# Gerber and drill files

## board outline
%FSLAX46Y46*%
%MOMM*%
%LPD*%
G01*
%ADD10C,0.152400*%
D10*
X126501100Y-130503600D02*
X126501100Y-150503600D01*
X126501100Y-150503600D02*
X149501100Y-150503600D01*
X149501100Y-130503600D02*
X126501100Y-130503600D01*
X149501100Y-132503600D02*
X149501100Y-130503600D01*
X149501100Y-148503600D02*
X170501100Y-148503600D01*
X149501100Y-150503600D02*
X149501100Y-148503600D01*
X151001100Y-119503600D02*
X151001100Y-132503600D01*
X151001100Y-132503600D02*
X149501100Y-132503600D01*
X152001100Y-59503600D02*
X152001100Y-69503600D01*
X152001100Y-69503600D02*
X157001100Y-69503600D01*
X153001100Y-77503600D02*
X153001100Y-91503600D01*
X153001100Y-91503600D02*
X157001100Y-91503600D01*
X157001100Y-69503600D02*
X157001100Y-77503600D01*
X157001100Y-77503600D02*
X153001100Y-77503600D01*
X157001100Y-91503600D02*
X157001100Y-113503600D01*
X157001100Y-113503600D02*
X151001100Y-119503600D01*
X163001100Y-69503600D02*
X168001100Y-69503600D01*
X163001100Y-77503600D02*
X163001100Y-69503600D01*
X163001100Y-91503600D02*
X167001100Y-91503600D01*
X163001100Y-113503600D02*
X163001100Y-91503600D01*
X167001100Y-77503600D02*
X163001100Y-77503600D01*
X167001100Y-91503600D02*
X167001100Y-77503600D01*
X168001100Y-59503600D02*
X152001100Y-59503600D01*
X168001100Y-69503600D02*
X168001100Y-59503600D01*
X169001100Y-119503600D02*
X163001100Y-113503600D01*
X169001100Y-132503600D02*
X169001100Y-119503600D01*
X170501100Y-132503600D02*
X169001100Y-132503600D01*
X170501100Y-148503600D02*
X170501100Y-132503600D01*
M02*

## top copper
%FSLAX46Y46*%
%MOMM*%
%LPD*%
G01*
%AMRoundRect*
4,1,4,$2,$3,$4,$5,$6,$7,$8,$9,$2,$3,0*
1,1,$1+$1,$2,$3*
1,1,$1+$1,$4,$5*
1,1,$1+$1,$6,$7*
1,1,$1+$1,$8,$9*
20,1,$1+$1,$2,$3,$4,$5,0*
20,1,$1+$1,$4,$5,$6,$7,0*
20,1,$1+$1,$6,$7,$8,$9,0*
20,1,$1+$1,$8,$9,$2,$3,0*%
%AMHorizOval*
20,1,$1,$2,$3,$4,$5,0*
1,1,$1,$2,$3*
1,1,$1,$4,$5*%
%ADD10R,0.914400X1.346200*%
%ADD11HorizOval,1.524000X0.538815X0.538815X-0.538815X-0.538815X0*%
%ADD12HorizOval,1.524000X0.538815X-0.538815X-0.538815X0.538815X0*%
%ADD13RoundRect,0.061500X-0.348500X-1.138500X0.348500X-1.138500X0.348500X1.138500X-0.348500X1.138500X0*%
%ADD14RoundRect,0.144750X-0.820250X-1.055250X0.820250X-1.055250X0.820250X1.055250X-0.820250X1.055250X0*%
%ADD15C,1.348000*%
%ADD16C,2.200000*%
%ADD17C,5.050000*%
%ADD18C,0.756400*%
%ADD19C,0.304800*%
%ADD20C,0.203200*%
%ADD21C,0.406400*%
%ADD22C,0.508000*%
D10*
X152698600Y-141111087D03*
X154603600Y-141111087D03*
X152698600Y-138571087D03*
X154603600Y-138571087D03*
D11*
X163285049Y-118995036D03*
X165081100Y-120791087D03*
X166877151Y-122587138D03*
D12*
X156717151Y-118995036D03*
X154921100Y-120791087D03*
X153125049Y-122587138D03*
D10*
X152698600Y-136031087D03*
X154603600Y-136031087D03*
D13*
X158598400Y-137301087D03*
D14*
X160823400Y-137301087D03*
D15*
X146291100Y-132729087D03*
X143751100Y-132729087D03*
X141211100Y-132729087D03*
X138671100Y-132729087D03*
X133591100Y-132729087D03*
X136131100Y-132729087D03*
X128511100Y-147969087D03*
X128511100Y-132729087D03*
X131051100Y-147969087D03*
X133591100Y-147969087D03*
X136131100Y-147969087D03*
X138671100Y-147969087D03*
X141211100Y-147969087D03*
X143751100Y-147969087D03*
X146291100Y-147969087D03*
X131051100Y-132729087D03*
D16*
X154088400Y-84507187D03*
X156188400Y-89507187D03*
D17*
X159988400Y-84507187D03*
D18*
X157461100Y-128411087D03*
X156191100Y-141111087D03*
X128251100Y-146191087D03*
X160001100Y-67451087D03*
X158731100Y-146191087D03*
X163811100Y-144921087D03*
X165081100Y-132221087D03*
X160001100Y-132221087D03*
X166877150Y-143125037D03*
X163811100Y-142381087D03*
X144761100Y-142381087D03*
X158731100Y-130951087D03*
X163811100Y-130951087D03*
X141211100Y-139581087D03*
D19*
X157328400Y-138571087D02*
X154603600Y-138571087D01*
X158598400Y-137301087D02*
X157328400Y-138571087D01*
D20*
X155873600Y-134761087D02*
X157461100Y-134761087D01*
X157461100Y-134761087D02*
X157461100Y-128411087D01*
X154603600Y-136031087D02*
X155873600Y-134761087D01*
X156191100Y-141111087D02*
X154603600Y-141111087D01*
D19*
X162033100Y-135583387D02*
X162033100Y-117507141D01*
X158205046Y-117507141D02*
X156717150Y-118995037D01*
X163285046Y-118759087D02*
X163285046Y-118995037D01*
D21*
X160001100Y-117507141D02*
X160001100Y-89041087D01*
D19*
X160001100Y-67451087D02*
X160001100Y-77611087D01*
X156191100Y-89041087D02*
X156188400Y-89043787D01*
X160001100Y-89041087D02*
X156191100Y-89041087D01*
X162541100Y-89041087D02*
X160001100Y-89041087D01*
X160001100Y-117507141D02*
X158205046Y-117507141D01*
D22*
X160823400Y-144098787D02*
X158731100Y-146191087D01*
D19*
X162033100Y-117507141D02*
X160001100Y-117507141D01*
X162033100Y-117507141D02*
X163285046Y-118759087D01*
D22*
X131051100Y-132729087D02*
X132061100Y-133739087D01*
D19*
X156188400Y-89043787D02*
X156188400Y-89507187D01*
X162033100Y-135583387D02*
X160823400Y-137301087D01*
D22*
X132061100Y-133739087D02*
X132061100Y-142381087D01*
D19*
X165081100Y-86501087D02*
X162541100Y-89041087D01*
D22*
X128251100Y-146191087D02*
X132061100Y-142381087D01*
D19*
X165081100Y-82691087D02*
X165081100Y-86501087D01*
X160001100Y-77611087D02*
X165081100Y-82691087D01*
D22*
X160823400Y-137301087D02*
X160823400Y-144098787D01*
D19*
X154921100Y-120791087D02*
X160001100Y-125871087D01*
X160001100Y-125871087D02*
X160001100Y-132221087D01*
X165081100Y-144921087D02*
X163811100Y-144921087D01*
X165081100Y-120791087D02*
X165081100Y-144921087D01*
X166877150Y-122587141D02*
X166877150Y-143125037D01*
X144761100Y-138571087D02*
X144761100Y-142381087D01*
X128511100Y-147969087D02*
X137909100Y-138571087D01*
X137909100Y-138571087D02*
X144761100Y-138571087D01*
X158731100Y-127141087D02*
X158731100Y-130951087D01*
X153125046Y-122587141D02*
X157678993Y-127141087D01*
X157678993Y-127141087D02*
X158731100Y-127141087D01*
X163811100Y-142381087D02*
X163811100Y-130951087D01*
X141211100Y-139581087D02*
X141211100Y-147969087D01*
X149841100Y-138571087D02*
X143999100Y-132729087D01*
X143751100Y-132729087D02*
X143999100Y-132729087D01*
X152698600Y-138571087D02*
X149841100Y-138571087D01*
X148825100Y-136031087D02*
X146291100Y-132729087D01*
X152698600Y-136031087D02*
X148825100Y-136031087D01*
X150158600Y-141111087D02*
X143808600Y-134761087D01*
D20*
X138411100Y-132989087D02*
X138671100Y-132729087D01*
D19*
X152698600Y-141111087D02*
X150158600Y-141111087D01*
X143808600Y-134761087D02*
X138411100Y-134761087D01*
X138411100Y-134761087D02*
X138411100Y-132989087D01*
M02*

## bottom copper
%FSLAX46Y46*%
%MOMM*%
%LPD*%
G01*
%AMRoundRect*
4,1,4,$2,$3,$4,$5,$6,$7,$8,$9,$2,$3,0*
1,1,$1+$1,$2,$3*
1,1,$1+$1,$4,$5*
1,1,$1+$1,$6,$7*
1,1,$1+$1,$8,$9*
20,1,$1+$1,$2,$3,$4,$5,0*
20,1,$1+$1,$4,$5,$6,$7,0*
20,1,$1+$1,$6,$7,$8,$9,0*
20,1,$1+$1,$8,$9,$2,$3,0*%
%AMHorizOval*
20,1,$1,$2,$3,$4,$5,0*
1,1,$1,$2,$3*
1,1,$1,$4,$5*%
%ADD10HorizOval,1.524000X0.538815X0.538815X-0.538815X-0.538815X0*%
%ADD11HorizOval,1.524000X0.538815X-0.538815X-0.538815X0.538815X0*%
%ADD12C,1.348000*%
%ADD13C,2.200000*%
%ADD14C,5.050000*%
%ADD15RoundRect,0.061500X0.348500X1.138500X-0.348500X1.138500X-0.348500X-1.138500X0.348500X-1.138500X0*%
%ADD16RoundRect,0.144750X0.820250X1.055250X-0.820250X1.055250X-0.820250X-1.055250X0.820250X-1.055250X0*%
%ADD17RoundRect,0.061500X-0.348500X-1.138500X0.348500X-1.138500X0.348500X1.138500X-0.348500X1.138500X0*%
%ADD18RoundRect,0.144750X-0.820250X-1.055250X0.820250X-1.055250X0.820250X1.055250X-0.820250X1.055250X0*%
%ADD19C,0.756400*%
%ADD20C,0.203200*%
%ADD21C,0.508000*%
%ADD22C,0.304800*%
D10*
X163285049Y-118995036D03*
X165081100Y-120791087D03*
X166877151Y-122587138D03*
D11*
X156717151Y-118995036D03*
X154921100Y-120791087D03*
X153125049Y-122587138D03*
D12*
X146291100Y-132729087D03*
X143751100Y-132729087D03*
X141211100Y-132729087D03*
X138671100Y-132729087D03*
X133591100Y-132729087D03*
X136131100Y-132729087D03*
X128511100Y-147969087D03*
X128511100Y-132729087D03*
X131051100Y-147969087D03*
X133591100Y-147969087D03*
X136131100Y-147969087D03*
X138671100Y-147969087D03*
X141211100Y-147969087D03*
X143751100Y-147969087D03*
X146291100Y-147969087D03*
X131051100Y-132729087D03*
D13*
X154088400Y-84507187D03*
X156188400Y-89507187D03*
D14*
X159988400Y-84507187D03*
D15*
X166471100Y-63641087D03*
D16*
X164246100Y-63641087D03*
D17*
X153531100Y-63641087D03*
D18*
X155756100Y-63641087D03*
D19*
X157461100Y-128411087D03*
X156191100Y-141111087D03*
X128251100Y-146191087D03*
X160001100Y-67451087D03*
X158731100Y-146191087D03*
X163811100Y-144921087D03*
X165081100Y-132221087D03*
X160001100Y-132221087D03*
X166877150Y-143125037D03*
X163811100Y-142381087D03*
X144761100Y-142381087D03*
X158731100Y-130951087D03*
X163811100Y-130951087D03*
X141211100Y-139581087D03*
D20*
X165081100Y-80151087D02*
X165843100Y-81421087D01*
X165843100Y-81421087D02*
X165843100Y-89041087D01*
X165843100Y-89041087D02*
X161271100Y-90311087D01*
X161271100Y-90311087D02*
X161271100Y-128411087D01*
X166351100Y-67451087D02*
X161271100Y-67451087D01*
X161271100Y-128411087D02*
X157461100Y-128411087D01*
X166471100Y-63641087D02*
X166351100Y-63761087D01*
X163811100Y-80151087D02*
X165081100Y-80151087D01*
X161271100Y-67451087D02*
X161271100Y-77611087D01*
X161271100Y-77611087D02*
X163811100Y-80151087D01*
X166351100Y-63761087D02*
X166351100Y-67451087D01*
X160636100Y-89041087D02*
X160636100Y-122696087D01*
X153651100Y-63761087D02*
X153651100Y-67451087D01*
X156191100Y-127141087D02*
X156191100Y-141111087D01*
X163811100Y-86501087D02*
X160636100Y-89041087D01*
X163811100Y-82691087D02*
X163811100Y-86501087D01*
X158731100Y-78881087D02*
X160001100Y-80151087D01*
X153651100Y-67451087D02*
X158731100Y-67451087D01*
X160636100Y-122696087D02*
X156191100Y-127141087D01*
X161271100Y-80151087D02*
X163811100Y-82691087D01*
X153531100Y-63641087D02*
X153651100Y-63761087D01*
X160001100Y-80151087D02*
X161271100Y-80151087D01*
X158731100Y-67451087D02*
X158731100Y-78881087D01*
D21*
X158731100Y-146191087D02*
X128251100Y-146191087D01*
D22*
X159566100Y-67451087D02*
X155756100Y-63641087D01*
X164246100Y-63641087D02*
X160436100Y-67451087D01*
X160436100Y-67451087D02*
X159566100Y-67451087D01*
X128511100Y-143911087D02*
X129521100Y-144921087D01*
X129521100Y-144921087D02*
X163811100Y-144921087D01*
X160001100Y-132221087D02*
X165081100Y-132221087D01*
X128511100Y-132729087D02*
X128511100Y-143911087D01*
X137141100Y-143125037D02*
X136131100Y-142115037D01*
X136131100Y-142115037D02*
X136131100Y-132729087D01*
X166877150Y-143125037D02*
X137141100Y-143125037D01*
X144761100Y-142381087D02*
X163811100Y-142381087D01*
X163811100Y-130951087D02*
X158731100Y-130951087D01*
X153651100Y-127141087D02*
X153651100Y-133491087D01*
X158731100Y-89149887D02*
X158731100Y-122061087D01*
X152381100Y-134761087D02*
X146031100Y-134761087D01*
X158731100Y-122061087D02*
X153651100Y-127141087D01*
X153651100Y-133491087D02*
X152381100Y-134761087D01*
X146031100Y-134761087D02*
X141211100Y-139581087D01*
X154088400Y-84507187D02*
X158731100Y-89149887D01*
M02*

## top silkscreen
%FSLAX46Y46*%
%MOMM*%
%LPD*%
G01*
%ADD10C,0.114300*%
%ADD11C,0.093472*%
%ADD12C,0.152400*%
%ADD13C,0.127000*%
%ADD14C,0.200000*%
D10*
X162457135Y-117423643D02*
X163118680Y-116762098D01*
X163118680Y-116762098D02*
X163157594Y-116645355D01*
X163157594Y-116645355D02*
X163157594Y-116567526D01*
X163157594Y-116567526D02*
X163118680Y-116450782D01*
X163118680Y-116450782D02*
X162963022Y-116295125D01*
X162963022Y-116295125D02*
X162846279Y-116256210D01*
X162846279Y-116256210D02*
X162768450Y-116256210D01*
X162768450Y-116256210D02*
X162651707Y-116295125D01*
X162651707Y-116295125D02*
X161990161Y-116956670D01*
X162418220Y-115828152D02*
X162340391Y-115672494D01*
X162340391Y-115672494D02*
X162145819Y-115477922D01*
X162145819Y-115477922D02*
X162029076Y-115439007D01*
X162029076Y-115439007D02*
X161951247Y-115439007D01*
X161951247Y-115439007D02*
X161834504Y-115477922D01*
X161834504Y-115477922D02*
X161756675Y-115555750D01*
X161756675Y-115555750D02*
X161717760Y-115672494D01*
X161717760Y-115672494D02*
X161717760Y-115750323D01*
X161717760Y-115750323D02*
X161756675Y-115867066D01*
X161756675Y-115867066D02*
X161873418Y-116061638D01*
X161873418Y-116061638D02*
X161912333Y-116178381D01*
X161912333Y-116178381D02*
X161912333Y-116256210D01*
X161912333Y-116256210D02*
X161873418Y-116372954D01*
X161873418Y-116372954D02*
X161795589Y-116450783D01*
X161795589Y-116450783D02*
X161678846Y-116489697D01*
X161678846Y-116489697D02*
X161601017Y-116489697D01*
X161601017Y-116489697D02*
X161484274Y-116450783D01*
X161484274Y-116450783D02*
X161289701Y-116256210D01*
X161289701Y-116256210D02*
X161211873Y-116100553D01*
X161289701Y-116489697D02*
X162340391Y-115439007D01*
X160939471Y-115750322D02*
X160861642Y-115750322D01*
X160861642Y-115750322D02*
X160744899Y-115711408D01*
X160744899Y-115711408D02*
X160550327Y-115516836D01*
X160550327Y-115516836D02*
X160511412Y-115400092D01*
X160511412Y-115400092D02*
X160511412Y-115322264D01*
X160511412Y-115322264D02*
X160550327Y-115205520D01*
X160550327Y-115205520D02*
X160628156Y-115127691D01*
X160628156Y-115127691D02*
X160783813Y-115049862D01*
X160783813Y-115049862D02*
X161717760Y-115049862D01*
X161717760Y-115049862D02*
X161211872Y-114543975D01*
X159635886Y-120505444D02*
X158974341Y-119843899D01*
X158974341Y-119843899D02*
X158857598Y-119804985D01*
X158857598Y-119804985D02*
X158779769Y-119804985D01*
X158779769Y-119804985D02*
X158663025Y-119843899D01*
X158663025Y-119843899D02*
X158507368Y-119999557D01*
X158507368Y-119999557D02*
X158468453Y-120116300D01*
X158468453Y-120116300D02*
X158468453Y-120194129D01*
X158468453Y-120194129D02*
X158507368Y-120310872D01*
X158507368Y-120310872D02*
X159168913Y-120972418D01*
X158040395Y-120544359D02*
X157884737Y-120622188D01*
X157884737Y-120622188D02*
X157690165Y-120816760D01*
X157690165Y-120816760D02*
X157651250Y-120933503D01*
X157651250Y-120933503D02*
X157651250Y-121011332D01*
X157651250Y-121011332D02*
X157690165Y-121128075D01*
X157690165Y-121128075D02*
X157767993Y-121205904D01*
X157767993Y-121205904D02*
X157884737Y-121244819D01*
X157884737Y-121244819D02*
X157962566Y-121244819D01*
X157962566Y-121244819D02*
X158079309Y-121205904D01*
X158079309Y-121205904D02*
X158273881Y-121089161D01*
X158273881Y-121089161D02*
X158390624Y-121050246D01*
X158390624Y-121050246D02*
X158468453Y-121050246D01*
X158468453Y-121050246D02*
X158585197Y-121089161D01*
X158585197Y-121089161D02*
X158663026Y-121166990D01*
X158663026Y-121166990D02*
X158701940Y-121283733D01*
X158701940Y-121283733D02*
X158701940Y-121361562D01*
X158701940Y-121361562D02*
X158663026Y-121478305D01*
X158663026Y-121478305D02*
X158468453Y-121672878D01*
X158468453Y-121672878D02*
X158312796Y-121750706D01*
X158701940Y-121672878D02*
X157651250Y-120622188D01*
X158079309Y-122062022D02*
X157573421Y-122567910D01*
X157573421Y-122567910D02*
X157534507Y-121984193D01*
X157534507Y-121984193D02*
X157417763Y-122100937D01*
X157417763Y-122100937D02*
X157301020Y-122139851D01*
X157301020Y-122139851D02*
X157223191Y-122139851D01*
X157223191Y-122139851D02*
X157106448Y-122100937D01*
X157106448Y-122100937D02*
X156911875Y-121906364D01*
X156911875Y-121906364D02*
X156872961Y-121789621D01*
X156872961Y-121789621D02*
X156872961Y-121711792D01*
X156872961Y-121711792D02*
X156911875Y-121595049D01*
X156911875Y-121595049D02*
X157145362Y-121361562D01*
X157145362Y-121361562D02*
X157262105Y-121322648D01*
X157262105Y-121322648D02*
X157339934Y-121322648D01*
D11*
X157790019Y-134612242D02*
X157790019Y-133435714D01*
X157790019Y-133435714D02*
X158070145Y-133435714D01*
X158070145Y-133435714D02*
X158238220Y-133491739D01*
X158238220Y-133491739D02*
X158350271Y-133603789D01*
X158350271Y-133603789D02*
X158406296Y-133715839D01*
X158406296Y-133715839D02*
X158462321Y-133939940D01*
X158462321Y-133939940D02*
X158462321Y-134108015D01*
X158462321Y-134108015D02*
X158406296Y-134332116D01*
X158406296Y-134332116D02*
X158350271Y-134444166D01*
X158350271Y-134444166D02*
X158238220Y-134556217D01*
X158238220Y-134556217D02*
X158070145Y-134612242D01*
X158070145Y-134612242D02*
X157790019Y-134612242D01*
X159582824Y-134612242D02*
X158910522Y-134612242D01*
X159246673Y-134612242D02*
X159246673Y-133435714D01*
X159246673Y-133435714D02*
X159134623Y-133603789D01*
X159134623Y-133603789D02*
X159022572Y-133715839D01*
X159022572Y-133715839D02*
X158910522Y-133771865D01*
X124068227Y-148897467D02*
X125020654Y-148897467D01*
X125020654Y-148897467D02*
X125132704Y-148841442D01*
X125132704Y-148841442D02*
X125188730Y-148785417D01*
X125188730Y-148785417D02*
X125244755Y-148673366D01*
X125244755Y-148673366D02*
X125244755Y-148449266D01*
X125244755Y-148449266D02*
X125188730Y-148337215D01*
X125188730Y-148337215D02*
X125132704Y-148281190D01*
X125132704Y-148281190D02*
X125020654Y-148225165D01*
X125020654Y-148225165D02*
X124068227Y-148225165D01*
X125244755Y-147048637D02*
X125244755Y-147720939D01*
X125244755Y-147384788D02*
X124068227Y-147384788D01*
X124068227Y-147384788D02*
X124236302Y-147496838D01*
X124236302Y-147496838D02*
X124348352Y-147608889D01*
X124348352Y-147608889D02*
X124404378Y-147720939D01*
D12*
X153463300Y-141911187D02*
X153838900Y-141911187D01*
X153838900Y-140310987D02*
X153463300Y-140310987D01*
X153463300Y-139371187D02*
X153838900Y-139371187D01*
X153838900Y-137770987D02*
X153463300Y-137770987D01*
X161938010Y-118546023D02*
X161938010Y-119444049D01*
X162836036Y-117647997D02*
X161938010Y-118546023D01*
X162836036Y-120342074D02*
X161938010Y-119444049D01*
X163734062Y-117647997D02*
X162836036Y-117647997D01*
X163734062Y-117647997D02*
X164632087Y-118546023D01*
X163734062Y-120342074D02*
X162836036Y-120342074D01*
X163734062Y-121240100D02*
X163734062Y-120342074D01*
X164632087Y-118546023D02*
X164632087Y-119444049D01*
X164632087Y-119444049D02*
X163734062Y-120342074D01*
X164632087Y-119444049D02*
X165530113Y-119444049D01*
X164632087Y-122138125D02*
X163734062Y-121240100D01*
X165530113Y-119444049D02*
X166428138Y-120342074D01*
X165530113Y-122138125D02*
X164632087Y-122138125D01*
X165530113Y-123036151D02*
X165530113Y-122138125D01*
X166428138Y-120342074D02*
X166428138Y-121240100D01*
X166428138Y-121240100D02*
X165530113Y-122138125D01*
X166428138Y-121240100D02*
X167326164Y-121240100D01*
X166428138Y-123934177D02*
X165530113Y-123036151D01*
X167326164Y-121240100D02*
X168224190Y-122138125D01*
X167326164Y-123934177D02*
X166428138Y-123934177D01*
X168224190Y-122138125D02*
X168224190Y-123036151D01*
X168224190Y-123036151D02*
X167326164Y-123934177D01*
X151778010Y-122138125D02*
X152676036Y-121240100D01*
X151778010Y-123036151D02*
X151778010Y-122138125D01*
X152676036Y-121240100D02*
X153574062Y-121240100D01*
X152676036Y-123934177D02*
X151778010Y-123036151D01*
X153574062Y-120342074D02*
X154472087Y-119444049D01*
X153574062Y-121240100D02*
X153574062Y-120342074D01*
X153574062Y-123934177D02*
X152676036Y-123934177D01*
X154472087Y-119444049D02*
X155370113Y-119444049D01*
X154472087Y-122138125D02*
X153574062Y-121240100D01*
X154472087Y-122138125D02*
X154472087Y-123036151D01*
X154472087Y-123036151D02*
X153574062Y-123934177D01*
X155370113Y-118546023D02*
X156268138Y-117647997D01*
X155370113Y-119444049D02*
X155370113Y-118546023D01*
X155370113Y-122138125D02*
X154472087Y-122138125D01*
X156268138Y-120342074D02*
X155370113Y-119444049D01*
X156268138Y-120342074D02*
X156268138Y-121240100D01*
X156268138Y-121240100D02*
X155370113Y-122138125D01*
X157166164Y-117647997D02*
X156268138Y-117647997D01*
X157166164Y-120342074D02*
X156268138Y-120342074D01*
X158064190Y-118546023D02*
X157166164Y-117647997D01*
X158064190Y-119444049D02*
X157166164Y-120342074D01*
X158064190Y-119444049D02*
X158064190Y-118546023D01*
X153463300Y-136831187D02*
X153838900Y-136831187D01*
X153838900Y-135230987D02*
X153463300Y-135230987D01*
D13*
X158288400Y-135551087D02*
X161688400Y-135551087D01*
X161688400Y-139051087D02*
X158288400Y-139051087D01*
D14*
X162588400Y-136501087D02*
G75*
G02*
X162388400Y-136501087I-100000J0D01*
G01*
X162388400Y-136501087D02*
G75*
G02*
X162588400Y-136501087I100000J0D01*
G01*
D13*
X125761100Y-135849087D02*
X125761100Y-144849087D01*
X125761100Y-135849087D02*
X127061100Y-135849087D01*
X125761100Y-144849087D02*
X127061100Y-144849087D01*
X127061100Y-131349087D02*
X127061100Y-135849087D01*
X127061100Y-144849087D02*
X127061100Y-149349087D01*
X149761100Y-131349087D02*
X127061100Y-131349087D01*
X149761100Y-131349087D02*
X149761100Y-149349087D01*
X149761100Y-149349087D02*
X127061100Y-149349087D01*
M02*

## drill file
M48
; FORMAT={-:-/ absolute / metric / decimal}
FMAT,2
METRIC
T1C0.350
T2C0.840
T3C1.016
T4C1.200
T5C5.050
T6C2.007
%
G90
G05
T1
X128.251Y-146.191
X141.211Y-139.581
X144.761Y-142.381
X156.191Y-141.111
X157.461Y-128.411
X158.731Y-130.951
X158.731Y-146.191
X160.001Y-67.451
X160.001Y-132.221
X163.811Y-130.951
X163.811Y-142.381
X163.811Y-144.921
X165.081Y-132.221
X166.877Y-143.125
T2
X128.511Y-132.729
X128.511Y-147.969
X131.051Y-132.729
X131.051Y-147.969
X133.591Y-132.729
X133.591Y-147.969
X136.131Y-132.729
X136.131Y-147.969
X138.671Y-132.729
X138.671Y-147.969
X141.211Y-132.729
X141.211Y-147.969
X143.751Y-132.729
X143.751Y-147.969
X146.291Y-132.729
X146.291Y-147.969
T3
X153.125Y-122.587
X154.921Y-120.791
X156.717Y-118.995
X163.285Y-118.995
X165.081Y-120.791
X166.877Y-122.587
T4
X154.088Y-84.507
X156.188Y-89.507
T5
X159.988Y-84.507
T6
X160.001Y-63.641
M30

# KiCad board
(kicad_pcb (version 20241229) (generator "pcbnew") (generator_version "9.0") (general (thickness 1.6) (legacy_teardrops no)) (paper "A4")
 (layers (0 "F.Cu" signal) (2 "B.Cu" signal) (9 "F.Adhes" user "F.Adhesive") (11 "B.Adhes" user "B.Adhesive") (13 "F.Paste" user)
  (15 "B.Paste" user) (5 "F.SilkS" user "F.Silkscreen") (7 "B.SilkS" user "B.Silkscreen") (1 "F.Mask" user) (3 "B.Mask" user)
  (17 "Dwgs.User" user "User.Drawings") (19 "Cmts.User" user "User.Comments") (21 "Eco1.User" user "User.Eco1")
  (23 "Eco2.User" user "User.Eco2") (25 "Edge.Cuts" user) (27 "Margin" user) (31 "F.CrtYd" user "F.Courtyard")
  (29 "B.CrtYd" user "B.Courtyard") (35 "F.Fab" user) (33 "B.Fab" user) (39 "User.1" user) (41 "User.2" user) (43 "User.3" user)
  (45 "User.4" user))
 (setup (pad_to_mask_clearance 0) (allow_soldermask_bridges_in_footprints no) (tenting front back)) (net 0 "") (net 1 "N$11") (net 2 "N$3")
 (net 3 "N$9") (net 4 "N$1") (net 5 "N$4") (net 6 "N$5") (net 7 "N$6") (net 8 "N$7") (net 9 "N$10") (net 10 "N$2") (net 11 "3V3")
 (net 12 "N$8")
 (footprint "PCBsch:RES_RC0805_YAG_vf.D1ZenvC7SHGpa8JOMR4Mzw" (layer "F.Cu") (at 153.6511 141.111087)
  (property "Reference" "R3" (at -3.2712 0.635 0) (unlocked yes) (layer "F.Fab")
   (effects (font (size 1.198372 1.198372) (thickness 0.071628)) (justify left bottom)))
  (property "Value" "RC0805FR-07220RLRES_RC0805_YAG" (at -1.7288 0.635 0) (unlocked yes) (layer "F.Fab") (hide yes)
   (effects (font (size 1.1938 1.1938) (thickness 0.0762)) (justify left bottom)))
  (fp_line (start -0.1878 0.8001) (end 0.1878 0.8001) (stroke (width 0.1524) (type solid)) (layer "F.SilkS"))
  (fp_line (start 0.1878 -0.8001) (end -0.1878 -0.8001) (stroke (width 0.1524) (type solid)) (layer "F.SilkS"))
  (pad "1" smd rect (at -0.9525 0) (size 0.9144 1.3462) (layers "F.Cu" "F.Mask" "F.Paste") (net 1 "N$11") (solder_mask_margin 0.1016)
   (solder_paste_margin 0) (thermal_bridge_angle 0))
  (pad "2" smd rect (at 0.9525 0) (size 0.9144 1.3462) (layers "F.Cu" "F.Mask" "F.Paste") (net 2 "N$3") (solder_mask_margin 0.1016)
   (solder_paste_margin 0) (thermal_bridge_angle 0))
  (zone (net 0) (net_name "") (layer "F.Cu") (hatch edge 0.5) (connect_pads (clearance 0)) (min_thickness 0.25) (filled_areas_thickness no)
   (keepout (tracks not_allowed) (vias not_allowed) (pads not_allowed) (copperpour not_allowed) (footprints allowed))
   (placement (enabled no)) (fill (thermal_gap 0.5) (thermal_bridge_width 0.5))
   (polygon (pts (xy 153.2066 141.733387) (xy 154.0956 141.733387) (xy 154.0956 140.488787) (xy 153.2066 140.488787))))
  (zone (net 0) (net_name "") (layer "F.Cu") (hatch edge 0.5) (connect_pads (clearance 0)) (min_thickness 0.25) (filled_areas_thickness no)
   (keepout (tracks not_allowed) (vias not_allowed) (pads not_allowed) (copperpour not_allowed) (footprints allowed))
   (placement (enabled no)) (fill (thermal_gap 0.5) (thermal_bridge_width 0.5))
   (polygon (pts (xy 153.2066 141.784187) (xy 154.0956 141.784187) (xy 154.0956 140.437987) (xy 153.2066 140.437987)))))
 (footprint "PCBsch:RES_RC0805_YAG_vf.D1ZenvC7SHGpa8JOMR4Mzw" (layer "F.Cu") (at 153.6511 138.571087)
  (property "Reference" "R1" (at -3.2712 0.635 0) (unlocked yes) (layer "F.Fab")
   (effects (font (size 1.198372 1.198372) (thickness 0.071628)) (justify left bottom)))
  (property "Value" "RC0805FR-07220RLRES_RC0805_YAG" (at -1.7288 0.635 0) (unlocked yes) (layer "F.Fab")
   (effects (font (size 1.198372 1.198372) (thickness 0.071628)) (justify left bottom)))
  (fp_line (start -0.1878 0.8001) (end 0.1878 0.8001) (stroke (width 0.1524) (type solid)) (layer "F.SilkS"))
  (fp_line (start 0.1878 -0.8001) (end -0.1878 -0.8001) (stroke (width 0.1524) (type solid)) (layer "F.SilkS"))
  (pad "1" smd rect (at -0.9525 0) (size 0.9144 1.3462) (layers "F.Cu" "F.Mask" "F.Paste") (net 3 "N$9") (solder_mask_margin 0.1016)
   (solder_paste_margin 0) (thermal_bridge_angle 0))
  (pad "2" smd rect (at 0.9525 0) (size 0.9144 1.3462) (layers "F.Cu" "F.Mask" "F.Paste") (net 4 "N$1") (solder_mask_margin 0.1016)
   (solder_paste_margin 0) (thermal_bridge_angle 0))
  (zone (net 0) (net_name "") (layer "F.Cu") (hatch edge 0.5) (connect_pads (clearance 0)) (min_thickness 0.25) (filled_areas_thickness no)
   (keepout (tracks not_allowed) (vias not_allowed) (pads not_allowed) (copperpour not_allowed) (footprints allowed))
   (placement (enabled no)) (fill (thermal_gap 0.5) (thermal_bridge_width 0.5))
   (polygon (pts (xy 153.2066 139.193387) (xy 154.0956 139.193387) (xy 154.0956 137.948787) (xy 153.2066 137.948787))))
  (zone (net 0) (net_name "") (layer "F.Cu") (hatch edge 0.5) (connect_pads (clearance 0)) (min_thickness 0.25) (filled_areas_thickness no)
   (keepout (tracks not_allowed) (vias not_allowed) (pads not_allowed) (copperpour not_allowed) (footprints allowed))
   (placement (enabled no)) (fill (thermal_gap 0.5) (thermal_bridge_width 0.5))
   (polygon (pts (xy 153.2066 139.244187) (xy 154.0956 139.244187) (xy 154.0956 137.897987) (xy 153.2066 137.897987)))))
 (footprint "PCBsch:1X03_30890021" (layer "F.Cu") (at 165.0811 120.791087 -45)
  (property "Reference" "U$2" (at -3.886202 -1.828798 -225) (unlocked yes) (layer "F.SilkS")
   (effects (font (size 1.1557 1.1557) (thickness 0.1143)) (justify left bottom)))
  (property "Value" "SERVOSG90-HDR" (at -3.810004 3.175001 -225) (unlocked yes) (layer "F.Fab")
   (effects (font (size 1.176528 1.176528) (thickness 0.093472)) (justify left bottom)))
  (fp_line (start -3.81 0.635) (end -3.175 1.270001) (stroke (width 0.1524) (type solid)) (layer "F.SilkS"))
  (fp_line (start -3.81 -0.635) (end -3.81 0.635) (stroke (width 0.1524) (type solid)) (layer "F.SilkS"))
  (fp_line (start -1.905 1.27) (end -3.175 1.270001) (stroke (width 0.1524) (type solid)) (layer "F.SilkS"))
  (fp_line (start -3.175 -1.270001) (end -3.81 -0.635) (stroke (width 0.1524) (type solid)) (layer "F.SilkS"))
  (fp_line (start -3.175 -1.270001) (end -1.905 -1.27) (stroke (width 0.1524) (type solid)) (layer "F.SilkS"))
  (fp_line (start -1.27 0.635) (end -1.905 1.27) (stroke (width 0.1524) (type solid)) (layer "F.SilkS"))
  (fp_line (start -0.635 1.27) (end -1.27 0.635) (stroke (width 0.1524) (type solid)) (layer "F.SilkS"))
  (fp_line (start -1.905 -1.27) (end -1.27 -0.635) (stroke (width 0.1524) (type solid)) (layer "F.SilkS"))
  (fp_line (start -1.27 -0.635) (end -1.27 0.635) (stroke (width 0.1524) (type solid)) (layer "F.SilkS"))
  (fp_line (start -1.27 -0.635) (end -0.635 -1.27) (stroke (width 0.1524) (type solid)) (layer "F.SilkS"))
  (fp_line (start 0.635 1.27) (end -0.635 1.27) (stroke (width 0.1524) (type solid)) (layer "F.SilkS"))
  (fp_line (start -0.635 -1.27) (end 0.635 -1.27) (stroke (width 0.1524) (type solid)) (layer "F.SilkS"))
  (fp_line (start 1.27 0.635) (end 0.635 1.27) (stroke (width 0.1524) (type solid)) (layer "F.SilkS"))
  (fp_line (start 1.905 1.27) (end 1.27 0.635) (stroke (width 0.1524) (type solid)) (layer "F.SilkS"))
  (fp_line (start 0.635 -1.27) (end 1.27 -0.635) (stroke (width 0.1524) (type solid)) (layer "F.SilkS"))
  (fp_line (start 1.27 -0.635) (end 1.27 0.635) (stroke (width 0.1524) (type solid)) (layer "F.SilkS"))
  (fp_line (start 1.27 -0.635) (end 1.905 -1.27) (stroke (width 0.1524) (type solid)) (layer "F.SilkS"))
  (fp_line (start 3.175 1.270001) (end 1.905 1.27) (stroke (width 0.1524) (type solid)) (layer "F.SilkS"))
  (fp_line (start 1.905 -1.27) (end 3.175 -1.270001) (stroke (width 0.1524) (type solid)) (layer "F.SilkS"))
  (fp_line (start 3.81 0.635) (end 3.175 1.270001) (stroke (width 0.1524) (type solid)) (layer "F.SilkS"))
  (fp_line (start 3.175 -1.270001) (end 3.81 -0.635) (stroke (width 0.1524) (type solid)) (layer "F.SilkS"))
  (fp_line (start 3.81 -0.635) (end 3.81 0.635) (stroke (width 0.1524) (type solid)) (layer "F.SilkS"))
  (pad "1" thru_hole oval (at -2.54 0 45) (size 3.048 1.524) (drill 1.016) (layers "*.Cu" "*.Mask") (remove_unused_layers no) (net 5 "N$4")
   (solder_mask_margin 0.1016) (thermal_bridge_angle 0))
  (pad "2" thru_hole oval (at 0 0 45) (size 3.048 1.524) (drill 1.016) (layers "*.Cu" "*.Mask") (remove_unused_layers no) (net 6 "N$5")
   (solder_mask_margin 0.1016) (thermal_bridge_angle 0))
  (pad "3" thru_hole oval (at 2.54 0 45) (size 3.048 1.524) (drill 1.016) (layers "*.Cu" "*.Mask") (remove_unused_layers no) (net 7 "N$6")
   (solder_mask_margin 0.1016) (thermal_bridge_angle 0)))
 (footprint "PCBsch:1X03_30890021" (layer "F.Cu") (at 154.9211 120.791087 -135)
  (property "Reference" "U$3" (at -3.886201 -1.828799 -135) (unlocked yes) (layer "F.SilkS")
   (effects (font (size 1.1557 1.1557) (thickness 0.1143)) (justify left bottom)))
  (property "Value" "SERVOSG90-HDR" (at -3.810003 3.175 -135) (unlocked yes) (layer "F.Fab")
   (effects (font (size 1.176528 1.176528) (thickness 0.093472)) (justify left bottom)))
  (fp_line (start 3.175 1.270001) (end 1.905 1.27) (stroke (width 0.1524) (type solid)) (layer "F.SilkS"))
  (fp_line (start 3.81 0.635) (end 3.175 1.270001) (stroke (width 0.1524) (type solid)) (layer "F.SilkS"))
  (fp_line (start 1.905 1.27) (end 1.27 0.635) (stroke (width 0.1524) (type solid)) (layer "F.SilkS"))
  (fp_line (start 3.81 -0.635) (end 3.81 0.635) (stroke (width 0.1524) (type solid)) (layer "F.SilkS"))
  (fp_line (start 0.635 1.27) (end -0.635 1.27) (stroke (width 0.1524) (type solid)) (layer "F.SilkS"))
  (fp_line (start 1.27 0.635) (end 0.635 1.27) (stroke (width 0.1524) (type solid)) (layer "F.SilkS"))
  (fp_line (start 3.175 -1.270001) (end 3.81 -0.635) (stroke (width 0.1524) (type solid)) (layer "F.SilkS"))
  (fp_line (start -0.635 1.27) (end -1.27 0.635) (stroke (width 0.1524) (type solid)) (layer "F.SilkS"))
  (fp_line (start 1.27 -0.635) (end 1.27 0.635) (stroke (width 0.1524) (type solid)) (layer "F.SilkS"))
  (fp_line (start 1.27 -0.635) (end 1.905 -1.27) (stroke (width 0.1524) (type solid)) (layer "F.SilkS"))
  (fp_line (start 1.905 -1.27) (end 3.175 -1.270001) (stroke (width 0.1524) (type solid)) (layer "F.SilkS"))
  (fp_line (start -1.905 1.27) (end -3.175 1.270001) (stroke (width 0.1524) (type solid)) (layer "F.SilkS"))
  (fp_line (start -1.27 0.635) (end -1.905 1.27) (stroke (width 0.1524) (type solid)) (layer "F.SilkS"))
  (fp_line (start 0.635 -1.27) (end 1.27 -0.635) (stroke (width 0.1524) (type solid)) (layer "F.SilkS"))
  (fp_line (start -1.27 -0.635) (end -1.27 0.635) (stroke (width 0.1524) (type solid)) (layer "F.SilkS"))
  (fp_line (start -1.27 -0.635) (end -0.635 -1.27) (stroke (width 0.1524) (type solid)) (layer "F.SilkS"))
  (fp_line (start -0.635 -1.27) (end 0.635 -1.27) (stroke (width 0.1524) (type solid)) (layer "F.SilkS"))
  (fp_line (start -3.81 0.635) (end -3.175 1.270001) (stroke (width 0.1524) (type solid)) (layer "F.SilkS"))
  (fp_line (start -1.905 -1.27) (end -1.27 -0.635) (stroke (width 0.1524) (type solid)) (layer "F.SilkS"))
  (fp_line (start -3.81 -0.635) (end -3.81 0.635) (stroke (width 0.1524) (type solid)) (layer "F.SilkS"))
  (fp_line (start -3.175 -1.270001) (end -1.905 -1.27) (stroke (width 0.1524) (type solid)) (layer "F.SilkS"))
  (fp_line (start -3.175 -1.270001) (end -3.81 -0.635) (stroke (width 0.1524) (type solid)) (layer "F.SilkS"))
  (pad "1" thru_hole oval (at -2.54 0 315) (size 3.048 1.524) (drill 1.016) (layers "*.Cu" "*.Mask") (remove_unused_layers no) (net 5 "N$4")
   (solder_mask_margin 0.1016) (thermal_bridge_angle 0))
  (pad "2" thru_hole oval (at 0 0 315) (size 3.048 1.524) (drill 1.016) (layers "*.Cu" "*.Mask") (remove_unused_layers no) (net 6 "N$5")
   (solder_mask_margin 0.1016) (thermal_bridge_angle 0))
  (pad "3" thru_hole oval (at 2.54 0 315) (size 3.048 1.524) (drill 1.016) (layers "*.Cu" "*.Mask") (remove_unused_layers no) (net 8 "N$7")
   (solder_mask_margin 0.1016) (thermal_bridge_angle 0)))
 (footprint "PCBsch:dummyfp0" (layer "F.Cu") (at 160.0011 63.641087)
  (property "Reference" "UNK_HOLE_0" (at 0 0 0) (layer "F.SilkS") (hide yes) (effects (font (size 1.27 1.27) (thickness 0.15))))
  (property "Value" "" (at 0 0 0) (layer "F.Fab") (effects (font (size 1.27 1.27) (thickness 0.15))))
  (pad "" np_thru_hole circle (at 0 0) (size 2.0066 2.0066) (drill 2.0066) (layers "*.Cu" "*.Mask")))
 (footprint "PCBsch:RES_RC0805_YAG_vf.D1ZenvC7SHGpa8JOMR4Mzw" (layer "F.Cu") (at 153.6511 136.031087)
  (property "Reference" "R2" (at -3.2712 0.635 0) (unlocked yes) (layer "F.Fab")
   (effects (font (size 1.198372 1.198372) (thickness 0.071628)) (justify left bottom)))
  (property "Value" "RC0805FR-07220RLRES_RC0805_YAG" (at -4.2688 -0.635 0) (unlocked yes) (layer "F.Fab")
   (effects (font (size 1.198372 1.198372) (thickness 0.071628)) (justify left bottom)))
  (fp_line (start -0.1878 0.8001) (end 0.1878 0.8001) (stroke (width 0.1524) (type solid)) (layer "F.SilkS"))
  (fp_line (start 0.1878 -0.8001) (end -0.1878 -0.8001) (stroke (width 0.1524) (type solid)) (layer "F.SilkS"))
  (pad "1" smd rect (at -0.9525 0) (size 0.9144 1.3462) (layers "F.Cu" "F.Mask" "F.Paste") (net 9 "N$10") (solder_mask_margin 0.1016)
   (solder_paste_margin 0) (thermal_bridge_angle 0))
  (pad "2" smd rect (at 0.9525 0) (size 0.9144 1.3462) (layers "F.Cu" "F.Mask" "F.Paste") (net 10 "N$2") (solder_mask_margin 0.1016)
   (solder_paste_margin 0) (thermal_bridge_angle 0))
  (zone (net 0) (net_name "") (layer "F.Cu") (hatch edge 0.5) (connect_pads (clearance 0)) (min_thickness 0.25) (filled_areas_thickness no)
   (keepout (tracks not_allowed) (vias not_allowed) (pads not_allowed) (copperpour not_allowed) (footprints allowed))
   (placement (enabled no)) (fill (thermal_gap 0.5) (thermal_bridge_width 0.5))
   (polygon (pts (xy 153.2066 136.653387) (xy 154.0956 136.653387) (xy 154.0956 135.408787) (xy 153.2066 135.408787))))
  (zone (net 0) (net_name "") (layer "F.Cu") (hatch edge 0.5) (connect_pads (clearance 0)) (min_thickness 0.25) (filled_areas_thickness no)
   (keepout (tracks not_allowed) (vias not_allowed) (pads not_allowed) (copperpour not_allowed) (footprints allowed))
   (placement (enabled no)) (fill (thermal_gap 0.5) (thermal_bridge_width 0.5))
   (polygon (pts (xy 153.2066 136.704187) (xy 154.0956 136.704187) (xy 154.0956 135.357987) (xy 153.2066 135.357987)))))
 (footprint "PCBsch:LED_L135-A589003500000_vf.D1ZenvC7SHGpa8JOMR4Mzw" (layer "F.Cu") (at 159.9884 137.301087)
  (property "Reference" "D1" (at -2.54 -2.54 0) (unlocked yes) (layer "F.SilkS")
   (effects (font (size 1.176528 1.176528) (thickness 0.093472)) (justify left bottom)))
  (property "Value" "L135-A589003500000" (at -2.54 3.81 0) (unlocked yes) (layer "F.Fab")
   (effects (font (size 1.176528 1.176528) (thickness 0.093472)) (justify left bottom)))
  (fp_line (start -1.7 -1.75) (end 1.7 -1.75) (stroke (width 0.127) (type solid)) (layer "F.SilkS"))
  (fp_line (start 1.7 1.75) (end -1.7 1.75) (stroke (width 0.127) (type solid)) (layer "F.SilkS"))
  (fp_circle (center 2.5 -0.8) (end 2.6 -0.8) (stroke (width 0.2) (type solid)) (fill no) (layer "F.SilkS"))
  (pad "A" smd roundrect (at -1.39 0) (size 0.82 2.4) (layers "F.Cu" "F.Paste") (roundrect_rratio 0.075) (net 4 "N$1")
   (solder_mask_margin 0.1016) (solder_paste_margin 0) (thermal_bridge_angle 0))
  (pad "C" smd roundrect (at 0.835 0) (size 1.93 2.4) (layers "F.Cu" "F.Paste") (roundrect_rratio 0.075) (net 5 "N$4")
   (solder_mask_margin 0.1016) (solder_paste_margin 0) (thermal_bridge_angle 0)))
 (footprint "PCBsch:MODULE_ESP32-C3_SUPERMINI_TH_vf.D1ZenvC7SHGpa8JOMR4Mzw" (layer "F.Cu") (at 138.4111 140.349087 90)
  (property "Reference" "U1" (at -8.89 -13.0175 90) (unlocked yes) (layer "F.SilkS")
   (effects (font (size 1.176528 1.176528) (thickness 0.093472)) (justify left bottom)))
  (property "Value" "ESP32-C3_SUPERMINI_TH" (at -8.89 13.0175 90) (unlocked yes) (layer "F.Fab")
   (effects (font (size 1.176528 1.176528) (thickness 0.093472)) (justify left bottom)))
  (fp_line (start 4.5 -12.65) (end -4.5 -12.65) (stroke (width 0.127) (type solid)) (layer "F.SilkS"))
  (fp_line (start 4.5 -12.65) (end 4.5 -11.35) (stroke (width 0.127) (type solid)) (layer "F.SilkS"))
  (fp_line (start -4.5 -12.65) (end -4.5 -11.35) (stroke (width 0.127) (type solid)) (layer "F.SilkS"))
  (fp_line (start 9 -11.35) (end 4.5 -11.35) (stroke (width 0.127) (type solid)) (layer "F.SilkS"))
  (fp_line (start -4.5 -11.35) (end -9 -11.35) (stroke (width 0.127) (type solid)) (layer "F.SilkS"))
  (fp_line (start 9 11.35) (end 9 -11.35) (stroke (width 0.127) (type solid)) (layer "F.SilkS"))
  (fp_line (start 9 11.35) (end -9 11.35) (stroke (width 0.127) (type solid)) (layer "F.SilkS"))
  (fp_line (start -9 11.35) (end -9 -11.35) (stroke (width 0.127) (type solid)) (layer "F.SilkS"))
  (pad "0" thru_hole circle (at 7.62 7.88 90) (size 1.348 1.348) (drill 0.84) (layers "*.Cu" "*.Mask") (remove_unused_layers no)
   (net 9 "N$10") (solder_mask_margin 0.1016) (thermal_bridge_angle 0))
  (pad "1" thru_hole circle (at 7.62 5.34 90) (size 1.348 1.348) (drill 0.84) (layers "*.Cu" "*.Mask") (remove_unused_layers no)
   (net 3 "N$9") (solder_mask_margin 0.1016) (thermal_bridge_angle 0))
  (pad "2" thru_hole circle (at 7.62 2.8 90) (size 1.348 1.348) (drill 0.84) (layers "*.Cu" "*.Mask") (remove_unused_layers no)
   (solder_mask_margin 0.1016) (thermal_bridge_angle 0))
  (pad "3" thru_hole circle (at 7.62 0.26 90) (size 1.348 1.348) (drill 0.84) (layers "*.Cu" "*.Mask") (remove_unused_layers no)
   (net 1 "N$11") (solder_mask_margin 0.1016) (thermal_bridge_angle 0))
  (pad "3.3" thru_hole circle (at 7.62 -4.82 90) (size 1.348 1.348) (drill 0.84) (layers "*.Cu" "*.Mask") (remove_unused_layers no)
   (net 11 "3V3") (solder_mask_margin 0.1016) (thermal_bridge_angle 0))
  (pad "4" thru_hole circle (at 7.62 -2.28 90) (size 1.348 1.348) (drill 0.84) (layers "*.Cu" "*.Mask") (remove_unused_layers no)
   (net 7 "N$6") (solder_mask_margin 0.1016) (thermal_bridge_angle 0))
  (pad "5" thru_hole circle (at -7.62 -9.9 90) (size 1.348 1.348) (drill 0.84) (layers "*.Cu" "*.Mask") (remove_unused_layers no)
   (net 8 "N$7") (solder_mask_margin 0.1016) (thermal_bridge_angle 0))
  (pad "5V" thru_hole circle (at 7.62 -9.9 90) (size 1.348 1.348) (drill 0.84) (layers "*.Cu" "*.Mask") (remove_unused_layers no)
   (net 6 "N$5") (solder_mask_margin 0.1016) (thermal_bridge_angle 0))
  (pad "6" thru_hole circle (at -7.62 -7.36 90) (size 1.348 1.348) (drill 0.84) (layers "*.Cu" "*.Mask") (remove_unused_layers no)
   (solder_mask_margin 0.1016) (thermal_bridge_angle 0))
  (pad "7" thru_hole circle (at -7.62 -4.82 90) (size 1.348 1.348) (drill 0.84) (layers "*.Cu" "*.Mask") (remove_unused_layers no)
   (solder_mask_margin 0.1016) (thermal_bridge_angle 0))
  (pad "8" thru_hole circle (at -7.62 -2.28 90) (size 1.348 1.348) (drill 0.84) (layers "*.Cu" "*.Mask") (remove_unused_layers no)
   (solder_mask_margin 0.1016) (thermal_bridge_angle 0))
  (pad "9" thru_hole circle (at -7.62 0.26 90) (size 1.348 1.348) (drill 0.84) (layers "*.Cu" "*.Mask") (remove_unused_layers no)
   (solder_mask_margin 0.1016) (thermal_bridge_angle 0))
  (pad "10" thru_hole circle (at -7.62 2.8 90) (size 1.348 1.348) (drill 0.84) (layers "*.Cu" "*.Mask") (remove_unused_layers no)
   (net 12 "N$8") (solder_mask_margin 0.1016) (thermal_bridge_angle 0))
  (pad "20" thru_hole circle (at -7.62 5.34 90) (size 1.348 1.348) (drill 0.84) (layers "*.Cu" "*.Mask") (remove_unused_layers no)
   (solder_mask_margin 0.1016) (thermal_bridge_angle 0))
  (pad "21" thru_hole circle (at -7.62 7.88 90) (size 1.348 1.348) (drill 0.84) (layers "*.Cu" "*.Mask") (remove_unused_layers no)
   (solder_mask_margin 0.1016) (thermal_bridge_angle 0))
  (pad "G" thru_hole circle (at 7.62 -7.36 90) (size 1.348 1.348) (drill 0.84) (layers "*.Cu" "*.Mask") (remove_unused_layers no)
   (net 5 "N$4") (solder_mask_margin 0.1016) (thermal_bridge_angle 0)))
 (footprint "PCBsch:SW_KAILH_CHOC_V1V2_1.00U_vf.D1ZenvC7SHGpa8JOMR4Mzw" (layer "B.Cu") (at 159.9884 84.507187 -90)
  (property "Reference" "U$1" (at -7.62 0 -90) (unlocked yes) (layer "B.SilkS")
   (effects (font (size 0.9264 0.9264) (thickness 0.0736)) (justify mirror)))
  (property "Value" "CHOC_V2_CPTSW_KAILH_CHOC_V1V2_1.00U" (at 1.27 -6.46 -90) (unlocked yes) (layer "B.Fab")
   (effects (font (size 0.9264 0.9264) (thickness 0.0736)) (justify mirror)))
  (pad "1" thru_hole circle (at 0 5.9 270) (size 2.2 2.2) (drill 1.2) (layers "*.Cu" "*.Mask") (remove_unused_layers no) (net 12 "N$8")
   (solder_mask_margin 0.1016) (thermal_bridge_angle 0))
  (pad "2" thru_hole circle (at 5 3.8 270) (size 2.2 2.2) (drill 1.2) (layers "*.Cu" "*.Mask") (remove_unused_layers no) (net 5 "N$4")
   (solder_mask_margin 0.1016) (thermal_bridge_angle 0))
  (pad "UN_3" thru_hole circle (at 0 0 270) (size 5.05 5.05) (drill 5.05) (layers "*.Cu" "*.Mask") (remove_unused_layers no)
   (solder_mask_margin 0.1016) (thermal_bridge_angle 0)))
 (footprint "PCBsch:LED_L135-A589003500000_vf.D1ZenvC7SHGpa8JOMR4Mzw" (layer "B.Cu") (at 165.0811 63.641087 180)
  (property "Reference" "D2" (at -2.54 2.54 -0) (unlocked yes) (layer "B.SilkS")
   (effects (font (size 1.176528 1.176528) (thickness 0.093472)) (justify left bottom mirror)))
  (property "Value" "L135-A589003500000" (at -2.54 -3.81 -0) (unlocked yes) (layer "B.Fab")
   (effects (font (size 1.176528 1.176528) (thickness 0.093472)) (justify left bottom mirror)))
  (pad "A" smd roundrect (at -1.39 0 180) (size 0.82 2.4) (layers "B.Cu" "B.Paste") (roundrect_rratio 0.075) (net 10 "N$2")
   (solder_mask_margin 0.1016) (solder_paste_margin 0) (thermal_bridge_angle 0))
  (pad "C" smd roundrect (at 0.835 0 180) (size 1.93 2.4) (layers "B.Cu" "B.Paste") (roundrect_rratio 0.075) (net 5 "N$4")
   (solder_mask_margin 0.1016) (solder_paste_margin 0) (thermal_bridge_angle 0)))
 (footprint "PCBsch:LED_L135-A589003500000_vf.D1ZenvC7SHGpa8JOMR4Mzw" (layer "B.Cu") (at 154.9211 63.641087)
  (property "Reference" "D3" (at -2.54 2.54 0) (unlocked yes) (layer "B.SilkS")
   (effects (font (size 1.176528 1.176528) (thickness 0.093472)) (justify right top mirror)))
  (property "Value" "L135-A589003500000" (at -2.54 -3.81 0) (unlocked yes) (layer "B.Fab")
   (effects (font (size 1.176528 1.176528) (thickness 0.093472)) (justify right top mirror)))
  (pad "A" smd roundrect (at -1.39 0) (size 0.82 2.4) (layers "B.Cu" "B.Paste") (roundrect_rratio 0.075) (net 2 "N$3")
   (solder_mask_margin 0.1016) (solder_paste_margin 0) (thermal_bridge_angle 0))
  (pad "C" smd roundrect (at 0.835 0) (size 1.93 2.4) (layers "B.Cu" "B.Paste") (roundrect_rratio 0.075) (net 5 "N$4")
   (solder_mask_margin 0.1016) (solder_paste_margin 0) (thermal_bridge_angle 0)))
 (gr_line (start 126.5011 130.5036) (end 126.5011 150.5036) (stroke (width 0.1524) (type solid)) (layer "Edge.Cuts"))
 (gr_line (start 126.5011 150.5036) (end 149.5011 150.5036) (stroke (width 0.1524) (type solid)) (layer "Edge.Cuts"))
 (gr_line (start 149.5011 130.5036) (end 126.5011 130.5036) (stroke (width 0.1524) (type solid)) (layer "Edge.Cuts"))
 (gr_line (start 149.5011 132.5036) (end 149.5011 130.5036) (stroke (width 0.1524) (type solid)) (layer "Edge.Cuts"))
 (gr_line (start 149.5011 148.5036) (end 170.5011 148.5036) (stroke (width 0.1524) (type solid)) (layer "Edge.Cuts"))
 (gr_line (start 149.5011 150.5036) (end 149.5011 148.5036) (stroke (width 0.1524) (type solid)) (layer "Edge.Cuts"))
 (gr_line (start 151.0011 119.5036) (end 151.0011 132.5036) (stroke (width 0.1524) (type solid)) (layer "Edge.Cuts"))
 (gr_line (start 151.0011 132.5036) (end 149.5011 132.5036) (stroke (width 0.1524) (type solid)) (layer "Edge.Cuts"))
 (gr_line (start 152.0011 59.5036) (end 152.0011 69.5036) (stroke (width 0.1524) (type solid)) (layer "Edge.Cuts"))
 (gr_line (start 152.0011 69.5036) (end 157.0011 69.5036) (stroke (width 0.1524) (type solid)) (layer "Edge.Cuts"))
 (gr_line (start 153.0011 77.5036) (end 153.0011 91.5036) (stroke (width 0.1524) (type solid)) (layer "Edge.Cuts"))
 (gr_line (start 153.0011 91.5036) (end 157.0011 91.5036) (stroke (width 0.1524) (type solid)) (layer "Edge.Cuts"))
 (gr_line (start 157.0011 69.5036) (end 157.0011 77.5036) (stroke (width 0.1524) (type solid)) (layer "Edge.Cuts"))
 (gr_line (start 157.0011 77.5036) (end 153.0011 77.5036) (stroke (width 0.1524) (type solid)) (layer "Edge.Cuts"))
 (gr_line (start 157.0011 91.5036) (end 157.0011 113.5036) (stroke (width 0.1524) (type solid)) (layer "Edge.Cuts"))
 (gr_line (start 157.0011 113.5036) (end 151.0011 119.5036) (stroke (width 0.1524) (type solid)) (layer "Edge.Cuts"))
 (gr_line (start 163.0011 69.5036) (end 168.0011 69.5036) (stroke (width 0.1524) (type solid)) (layer "Edge.Cuts"))
 (gr_line (start 163.0011 77.5036) (end 163.0011 69.5036) (stroke (width 0.1524) (type solid)) (layer "Edge.Cuts"))
 (gr_line (start 163.0011 91.5036) (end 167.0011 91.5036) (stroke (width 0.1524) (type solid)) (layer "Edge.Cuts"))
 (gr_line (start 163.0011 113.5036) (end 163.0011 91.5036) (stroke (width 0.1524) (type solid)) (layer "Edge.Cuts"))
 (gr_line (start 167.0011 77.5036) (end 163.0011 77.5036) (stroke (width 0.1524) (type solid)) (layer "Edge.Cuts"))
 (gr_line (start 167.0011 91.5036) (end 167.0011 77.5036) (stroke (width 0.1524) (type solid)) (layer "Edge.Cuts"))
 (gr_line (start 168.0011 59.5036) (end 152.0011 59.5036) (stroke (width 0.1524) (type solid)) (layer "Edge.Cuts"))
 (gr_line (start 168.0011 69.5036) (end 168.0011 59.5036) (stroke (width 0.1524) (type solid)) (layer "Edge.Cuts"))
 (gr_line (start 169.0011 119.5036) (end 163.0011 113.5036) (stroke (width 0.1524) (type solid)) (layer "Edge.Cuts"))
 (gr_line (start 169.0011 132.5036) (end 169.0011 119.5036) (stroke (width 0.1524) (type solid)) (layer "Edge.Cuts"))
 (gr_line (start 170.5011 132.5036) (end 169.0011 132.5036) (stroke (width 0.1524) (type solid)) (layer "Edge.Cuts"))
 (gr_line (start 170.5011 148.5036) (end 170.5011 132.5036) (stroke (width 0.1524) (type solid)) (layer "Edge.Cuts"))
 (segment (start 157.3284 138.571087) (end 154.6036 138.571087) (width 0.3048) (layer "F.Cu") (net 4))
 (segment (start 158.5984 137.301087) (end 157.3284 138.571087) (width 0.3048) (layer "F.Cu") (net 4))
 (segment (start 155.8736 134.761087) (end 157.4611 134.761087) (width 0.2032) (layer "F.Cu") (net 10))
 (segment (start 157.4611 134.761087) (end 157.4611 128.411087) (width 0.2032) (layer "F.Cu") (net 10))
 (segment (start 154.6036 136.031087) (end 155.8736 134.761087) (width 0.2032) (layer "F.Cu") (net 10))
 (via (at 157.4611 128.411087) (size 0.7564) (drill 0.35) (layers "F.Cu" "B.Cu") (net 10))
 (segment (start 165.0811 80.151087) (end 165.8431 81.421087) (width 0.2032) (layer "B.Cu") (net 10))
 (segment (start 165.8431 81.421087) (end 165.8431 89.041087) (width 0.2032) (layer "B.Cu") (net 10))
 (segment (start 165.8431 89.041087) (end 161.2711 90.311087) (width 0.2032) (layer "B.Cu") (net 10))
 (segment (start 161.2711 90.311087) (end 161.2711 128.411087) (width 0.2032) (layer "B.Cu") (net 10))
 (segment (start 166.3511 67.451087) (end 161.2711 67.451087) (width 0.2032) (layer "B.Cu") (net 10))
 (segment (start 161.2711 128.411087) (end 157.4611 128.411087) (width 0.2032) (layer "B.Cu") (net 10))
 (segment (start 166.4711 63.641087) (end 166.3511 63.761087) (width 0.2032) (layer "B.Cu") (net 10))
 (segment (start 163.8111 80.151087) (end 165.0811 80.151087) (width 0.2032) (layer "B.Cu") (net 10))
 (segment (start 161.2711 67.451087) (end 161.2711 77.611087) (width 0.2032) (layer "B.Cu") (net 10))
 (segment (start 161.2711 77.611087) (end 163.8111 80.151087) (width 0.2032) (layer "B.Cu") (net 10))
 (segment (start 166.3511 63.761087) (end 166.3511 67.451087) (width 0.2032) (layer "B.Cu") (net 10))
 (segment (start 156.1911 141.111087) (end 154.6036 141.111087) (width 0.2032) (layer "F.Cu") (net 2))
 (via (at 156.1911 141.111087) (size 0.7564) (drill 0.35) (layers "F.Cu" "B.Cu") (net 2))
 (segment (start 160.6361 89.041087) (end 160.6361 122.696087) (width 0.2032) (layer "B.Cu") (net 2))
 (segment (start 153.6511 63.761087) (end 153.6511 67.451087) (width 0.2032) (layer "B.Cu") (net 2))
 (segment (start 156.1911 127.141087) (end 156.1911 141.111087) (width 0.2032) (layer "B.Cu") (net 2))
 (segment (start 163.8111 86.501087) (end 160.6361 89.041087) (width 0.2032) (layer "B.Cu") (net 2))
 (segment (start 163.8111 82.691087) (end 163.8111 86.501087) (width 0.2032) (layer "B.Cu") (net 2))
 (segment (start 158.7311 78.881087) (end 160.0011 80.151087) (width 0.2032) (layer "B.Cu") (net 2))
 (segment (start 153.6511 67.451087) (end 158.7311 67.451087) (width 0.2032) (layer "B.Cu") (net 2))
 (segment (start 160.6361 122.696087) (end 156.1911 127.141087) (width 0.2032) (layer "B.Cu") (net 2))
 (segment (start 161.2711 80.151087) (end 163.8111 82.691087) (width 0.2032) (layer "B.Cu") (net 2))
 (segment (start 153.5311 63.641087) (end 153.6511 63.761087) (width 0.2032) (layer "B.Cu") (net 2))
 (segment (start 160.0011 80.151087) (end 161.2711 80.151087) (width 0.2032) (layer "B.Cu") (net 2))
 (segment (start 158.7311 67.451087) (end 158.7311 78.881087) (width 0.2032) (layer "B.Cu") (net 2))
 (segment (start 162.0331 135.583387) (end 162.0331 117.507141) (width 0.3048) (layer "F.Cu") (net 5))
 (segment (start 158.205046 117.507141) (end 156.71715 118.995037) (width 0.3048) (layer "F.Cu") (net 5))
 (segment (start 163.285046 118.759087) (end 163.285046 118.995037) (width 0.3048) (layer "F.Cu") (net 5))
 (segment (start 160.0011 117.507141) (end 160.0011 89.041087) (width 0.4064) (layer "F.Cu") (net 5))
 (segment (start 160.0011 67.451087) (end 160.0011 77.611087) (width 0.3048) (layer "F.Cu") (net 5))
 (segment (start 156.1911 89.041087) (end 156.1884 89.043787) (width 0.3048) (layer "F.Cu") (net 5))
 (segment (start 160.0011 89.041087) (end 156.1911 89.041087) (width 0.3048) (layer "F.Cu") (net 5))
 (segment (start 162.5411 89.041087) (end 160.0011 89.041087) (width 0.3048) (layer "F.Cu") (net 5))
 (segment (start 160.0011 117.507141) (end 158.205046 117.507141) (width 0.3048) (layer "F.Cu") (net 5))
 (segment (start 160.8234 144.098787) (end 158.7311 146.191087) (width 0.508) (layer "F.Cu") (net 5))
 (segment (start 162.0331 117.507141) (end 160.0011 117.507141) (width 0.3048) (layer "F.Cu") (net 5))
 (segment (start 162.0331 117.507141) (end 163.285046 118.759087) (width 0.3048) (layer "F.Cu") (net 5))
 (segment (start 131.0511 132.729087) (end 132.0611 133.739087) (width 0.508) (layer "F.Cu") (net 5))
 (segment (start 156.1884 89.043787) (end 156.1884 89.507187) (width 0.3048) (layer "F.Cu") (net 5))
 (segment (start 162.0331 135.583387) (end 160.8234 137.301087) (width 0.3048) (layer "F.Cu") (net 5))
 (segment (start 132.0611 133.739087) (end 132.0611 142.381087) (width 0.508) (layer "F.Cu") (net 5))
 (segment (start 165.0811 86.501087) (end 162.5411 89.041087) (width 0.3048) (layer "F.Cu") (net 5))
 (segment (start 128.2511 146.191087) (end 132.0611 142.381087) (width 0.508) (layer "F.Cu") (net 5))
 (segment (start 165.0811 82.691087) (end 165.0811 86.501087) (width 0.3048) (layer "F.Cu") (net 5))
 (segment (start 160.0011 77.611087) (end 165.0811 82.691087) (width 0.3048) (layer "F.Cu") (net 5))
 (segment (start 160.8234 137.301087) (end 160.8234 144.098787) (width 0.508) (layer "F.Cu") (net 5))
 (via (at 128.2511 146.191087) (size 0.7564) (drill 0.35) (layers "F.Cu" "B.Cu") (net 5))
 (via (at 160.0011 67.451087) (size 0.7564) (drill 0.35) (layers "F.Cu" "B.Cu") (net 5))
 (via (at 158.7311 146.191087) (size 0.7564) (drill 0.35) (layers "F.Cu" "B.Cu") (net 5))
 (segment (start 158.7311 146.191087) (end 128.2511 146.191087) (width 0.508) (layer "B.Cu") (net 5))
 (segment (start 159.5661 67.451087) (end 155.7561 63.641087) (width 0.3048) (layer "B.Cu") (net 5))
 (segment (start 164.2461 63.641087) (end 160.4361 67.451087) (width 0.3048) (layer "B.Cu") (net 5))
 (segment (start 160.4361 67.451087) (end 159.5661 67.451087) (width 0.3048) (layer "B.Cu") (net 5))
 (segment (start 154.9211 120.791087) (end 160.0011 125.871087) (width 0.3048) (layer "F.Cu") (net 6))
 (segment (start 160.0011 125.871087) (end 160.0011 132.221087) (width 0.3048) (layer "F.Cu") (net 6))
 (segment (start 165.0811 144.921087) (end 163.8111 144.921087) (width 0.3048) (layer "F.Cu") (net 6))
 (segment (start 165.0811 120.791087) (end 165.0811 144.921087) (width 0.3048) (layer "F.Cu") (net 6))
 (via (at 163.8111 144.921087) (size 0.7564) (drill 0.35) (layers "F.Cu" "B.Cu") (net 6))
 (via (at 165.0811 132.221087) (size 0.7564) (drill 0.35) (layers "F.Cu" "B.Cu") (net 6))
 (via (at 160.0011 132.221087) (size 0.7564) (drill 0.35) (layers "F.Cu" "B.Cu") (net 6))
 (segment (start 128.5111 143.911087) (end 129.5211 144.921087) (width 0.3048) (layer "B.Cu") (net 6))
 (segment (start 129.5211 144.921087) (end 163.8111 144.921087) (width 0.3048) (layer "B.Cu") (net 6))
 (segment (start 160.0011 132.221087) (end 165.0811 132.221087) (width 0.3048) (layer "B.Cu") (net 6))
 (segment (start 128.5111 132.729087) (end 128.5111 143.911087) (width 0.3048) (layer "B.Cu") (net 6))
 (segment (start 166.87715 122.587141) (end 166.87715 143.125037) (width 0.3048) (layer "F.Cu") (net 7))
 (via (at 166.87715 143.125037) (size 0.7564) (drill 0.35) (layers "F.Cu" "B.Cu") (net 7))
 (segment (start 137.1411 143.125037) (end 136.1311 142.115037) (width 0.3048) (layer "B.Cu") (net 7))
 (segment (start 136.1311 142.115037) (end 136.1311 132.729087) (width 0.3048) (layer "B.Cu") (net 7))
 (segment (start 166.87715 143.125037) (end 137.1411 143.125037) (width 0.3048) (layer "B.Cu") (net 7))
 (segment (start 144.7611 138.571087) (end 144.7611 142.381087) (width 0.3048) (layer "F.Cu") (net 8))
 (segment (start 128.5111 147.969087) (end 137.9091 138.571087) (width 0.3048) (layer "F.Cu") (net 8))
 (segment (start 137.9091 138.571087) (end 144.7611 138.571087) (width 0.3048) (layer "F.Cu") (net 8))
 (segment (start 158.7311 127.141087) (end 158.7311 130.951087) (width 0.3048) (layer "F.Cu") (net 8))
 (segment (start 153.125046 122.587141) (end 157.678993 127.141087) (width 0.3048) (layer "F.Cu") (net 8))
 (segment (start 157.678993 127.141087) (end 158.7311 127.141087) (width 0.3048) (layer "F.Cu") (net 8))
 (segment (start 163.8111 142.381087) (end 163.8111 130.951087) (width 0.3048) (layer "F.Cu") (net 8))
 (via (at 163.8111 142.381087) (size 0.7564) (drill 0.35) (layers "F.Cu" "B.Cu") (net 8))
 (via (at 144.7611 142.381087) (size 0.7564) (drill 0.35) (layers "F.Cu" "B.Cu") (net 8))
 (via (at 158.7311 130.951087) (size 0.7564) (drill 0.35) (layers "F.Cu" "B.Cu") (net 8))
 (via (at 163.8111 130.951087) (size 0.7564) (drill 0.35) (layers "F.Cu" "B.Cu") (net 8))
 (segment (start 144.7611 142.381087) (end 163.8111 142.381087) (width 0.3048) (layer "B.Cu") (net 8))
 (segment (start 163.8111 130.951087) (end 158.7311 130.951087) (width 0.3048) (layer "B.Cu") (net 8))
 (segment (start 141.2111 139.581087) (end 141.2111 147.969087) (width 0.3048) (layer "F.Cu") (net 12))
 (via (at 141.2111 139.581087) (size 0.7564) (drill 0.35) (layers "F.Cu" "B.Cu") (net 12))
 (segment (start 153.6511 127.141087) (end 153.6511 133.491087) (width 0.3048) (layer "B.Cu") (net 12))
 (segment (start 158.7311 89.149887) (end 158.7311 122.061087) (width 0.3048) (layer "B.Cu") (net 12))
 (segment (start 152.3811 134.761087) (end 146.0311 134.761087) (width 0.3048) (layer "B.Cu") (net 12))
 (segment (start 158.7311 122.061087) (end 153.6511 127.141087) (width 0.3048) (layer "B.Cu") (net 12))
 (segment (start 153.6511 133.491087) (end 152.3811 134.761087) (width 0.3048) (layer "B.Cu") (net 12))
 (segment (start 146.0311 134.761087) (end 141.2111 139.581087) (width 0.3048) (layer "B.Cu") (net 12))
 (segment (start 154.0884 84.507187) (end 158.7311 89.149887) (width 0.3048) (layer "B.Cu") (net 12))
 (segment (start 149.8411 138.571087) (end 143.9991 132.729087) (width 0.3048) (layer "F.Cu") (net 3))
 (segment (start 143.7511 132.729087) (end 143.9991 132.729087) (width 0.3048) (layer "F.Cu") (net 3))
 (segment (start 152.6986 138.571087) (end 149.8411 138.571087) (width 0.3048) (layer "F.Cu") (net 3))
 (segment (start 148.8251 136.031087) (end 146.2911 132.729087) (width 0.3048) (layer "F.Cu") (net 9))
 (segment (start 152.6986 136.031087) (end 148.8251 136.031087) (width 0.3048) (layer "F.Cu") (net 9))
 (segment (start 150.1586 141.111087) (end 143.8086 134.761087) (width 0.3048) (layer "F.Cu") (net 1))
 (segment (start 138.4111 132.989087) (end 138.6711 132.729087) (width 0.2032) (layer "F.Cu") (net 1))
 (segment (start 152.6986 141.111087) (end 150.1586 141.111087) (width 0.3048) (layer "F.Cu") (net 1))
 (segment (start 143.8086 134.761087) (end 138.4111 134.761087) (width 0.3048) (layer "F.Cu") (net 1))
 (segment (start 138.4111 134.761087) (end 138.4111 132.989087) (width 0.3048) (layer "F.Cu") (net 1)))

